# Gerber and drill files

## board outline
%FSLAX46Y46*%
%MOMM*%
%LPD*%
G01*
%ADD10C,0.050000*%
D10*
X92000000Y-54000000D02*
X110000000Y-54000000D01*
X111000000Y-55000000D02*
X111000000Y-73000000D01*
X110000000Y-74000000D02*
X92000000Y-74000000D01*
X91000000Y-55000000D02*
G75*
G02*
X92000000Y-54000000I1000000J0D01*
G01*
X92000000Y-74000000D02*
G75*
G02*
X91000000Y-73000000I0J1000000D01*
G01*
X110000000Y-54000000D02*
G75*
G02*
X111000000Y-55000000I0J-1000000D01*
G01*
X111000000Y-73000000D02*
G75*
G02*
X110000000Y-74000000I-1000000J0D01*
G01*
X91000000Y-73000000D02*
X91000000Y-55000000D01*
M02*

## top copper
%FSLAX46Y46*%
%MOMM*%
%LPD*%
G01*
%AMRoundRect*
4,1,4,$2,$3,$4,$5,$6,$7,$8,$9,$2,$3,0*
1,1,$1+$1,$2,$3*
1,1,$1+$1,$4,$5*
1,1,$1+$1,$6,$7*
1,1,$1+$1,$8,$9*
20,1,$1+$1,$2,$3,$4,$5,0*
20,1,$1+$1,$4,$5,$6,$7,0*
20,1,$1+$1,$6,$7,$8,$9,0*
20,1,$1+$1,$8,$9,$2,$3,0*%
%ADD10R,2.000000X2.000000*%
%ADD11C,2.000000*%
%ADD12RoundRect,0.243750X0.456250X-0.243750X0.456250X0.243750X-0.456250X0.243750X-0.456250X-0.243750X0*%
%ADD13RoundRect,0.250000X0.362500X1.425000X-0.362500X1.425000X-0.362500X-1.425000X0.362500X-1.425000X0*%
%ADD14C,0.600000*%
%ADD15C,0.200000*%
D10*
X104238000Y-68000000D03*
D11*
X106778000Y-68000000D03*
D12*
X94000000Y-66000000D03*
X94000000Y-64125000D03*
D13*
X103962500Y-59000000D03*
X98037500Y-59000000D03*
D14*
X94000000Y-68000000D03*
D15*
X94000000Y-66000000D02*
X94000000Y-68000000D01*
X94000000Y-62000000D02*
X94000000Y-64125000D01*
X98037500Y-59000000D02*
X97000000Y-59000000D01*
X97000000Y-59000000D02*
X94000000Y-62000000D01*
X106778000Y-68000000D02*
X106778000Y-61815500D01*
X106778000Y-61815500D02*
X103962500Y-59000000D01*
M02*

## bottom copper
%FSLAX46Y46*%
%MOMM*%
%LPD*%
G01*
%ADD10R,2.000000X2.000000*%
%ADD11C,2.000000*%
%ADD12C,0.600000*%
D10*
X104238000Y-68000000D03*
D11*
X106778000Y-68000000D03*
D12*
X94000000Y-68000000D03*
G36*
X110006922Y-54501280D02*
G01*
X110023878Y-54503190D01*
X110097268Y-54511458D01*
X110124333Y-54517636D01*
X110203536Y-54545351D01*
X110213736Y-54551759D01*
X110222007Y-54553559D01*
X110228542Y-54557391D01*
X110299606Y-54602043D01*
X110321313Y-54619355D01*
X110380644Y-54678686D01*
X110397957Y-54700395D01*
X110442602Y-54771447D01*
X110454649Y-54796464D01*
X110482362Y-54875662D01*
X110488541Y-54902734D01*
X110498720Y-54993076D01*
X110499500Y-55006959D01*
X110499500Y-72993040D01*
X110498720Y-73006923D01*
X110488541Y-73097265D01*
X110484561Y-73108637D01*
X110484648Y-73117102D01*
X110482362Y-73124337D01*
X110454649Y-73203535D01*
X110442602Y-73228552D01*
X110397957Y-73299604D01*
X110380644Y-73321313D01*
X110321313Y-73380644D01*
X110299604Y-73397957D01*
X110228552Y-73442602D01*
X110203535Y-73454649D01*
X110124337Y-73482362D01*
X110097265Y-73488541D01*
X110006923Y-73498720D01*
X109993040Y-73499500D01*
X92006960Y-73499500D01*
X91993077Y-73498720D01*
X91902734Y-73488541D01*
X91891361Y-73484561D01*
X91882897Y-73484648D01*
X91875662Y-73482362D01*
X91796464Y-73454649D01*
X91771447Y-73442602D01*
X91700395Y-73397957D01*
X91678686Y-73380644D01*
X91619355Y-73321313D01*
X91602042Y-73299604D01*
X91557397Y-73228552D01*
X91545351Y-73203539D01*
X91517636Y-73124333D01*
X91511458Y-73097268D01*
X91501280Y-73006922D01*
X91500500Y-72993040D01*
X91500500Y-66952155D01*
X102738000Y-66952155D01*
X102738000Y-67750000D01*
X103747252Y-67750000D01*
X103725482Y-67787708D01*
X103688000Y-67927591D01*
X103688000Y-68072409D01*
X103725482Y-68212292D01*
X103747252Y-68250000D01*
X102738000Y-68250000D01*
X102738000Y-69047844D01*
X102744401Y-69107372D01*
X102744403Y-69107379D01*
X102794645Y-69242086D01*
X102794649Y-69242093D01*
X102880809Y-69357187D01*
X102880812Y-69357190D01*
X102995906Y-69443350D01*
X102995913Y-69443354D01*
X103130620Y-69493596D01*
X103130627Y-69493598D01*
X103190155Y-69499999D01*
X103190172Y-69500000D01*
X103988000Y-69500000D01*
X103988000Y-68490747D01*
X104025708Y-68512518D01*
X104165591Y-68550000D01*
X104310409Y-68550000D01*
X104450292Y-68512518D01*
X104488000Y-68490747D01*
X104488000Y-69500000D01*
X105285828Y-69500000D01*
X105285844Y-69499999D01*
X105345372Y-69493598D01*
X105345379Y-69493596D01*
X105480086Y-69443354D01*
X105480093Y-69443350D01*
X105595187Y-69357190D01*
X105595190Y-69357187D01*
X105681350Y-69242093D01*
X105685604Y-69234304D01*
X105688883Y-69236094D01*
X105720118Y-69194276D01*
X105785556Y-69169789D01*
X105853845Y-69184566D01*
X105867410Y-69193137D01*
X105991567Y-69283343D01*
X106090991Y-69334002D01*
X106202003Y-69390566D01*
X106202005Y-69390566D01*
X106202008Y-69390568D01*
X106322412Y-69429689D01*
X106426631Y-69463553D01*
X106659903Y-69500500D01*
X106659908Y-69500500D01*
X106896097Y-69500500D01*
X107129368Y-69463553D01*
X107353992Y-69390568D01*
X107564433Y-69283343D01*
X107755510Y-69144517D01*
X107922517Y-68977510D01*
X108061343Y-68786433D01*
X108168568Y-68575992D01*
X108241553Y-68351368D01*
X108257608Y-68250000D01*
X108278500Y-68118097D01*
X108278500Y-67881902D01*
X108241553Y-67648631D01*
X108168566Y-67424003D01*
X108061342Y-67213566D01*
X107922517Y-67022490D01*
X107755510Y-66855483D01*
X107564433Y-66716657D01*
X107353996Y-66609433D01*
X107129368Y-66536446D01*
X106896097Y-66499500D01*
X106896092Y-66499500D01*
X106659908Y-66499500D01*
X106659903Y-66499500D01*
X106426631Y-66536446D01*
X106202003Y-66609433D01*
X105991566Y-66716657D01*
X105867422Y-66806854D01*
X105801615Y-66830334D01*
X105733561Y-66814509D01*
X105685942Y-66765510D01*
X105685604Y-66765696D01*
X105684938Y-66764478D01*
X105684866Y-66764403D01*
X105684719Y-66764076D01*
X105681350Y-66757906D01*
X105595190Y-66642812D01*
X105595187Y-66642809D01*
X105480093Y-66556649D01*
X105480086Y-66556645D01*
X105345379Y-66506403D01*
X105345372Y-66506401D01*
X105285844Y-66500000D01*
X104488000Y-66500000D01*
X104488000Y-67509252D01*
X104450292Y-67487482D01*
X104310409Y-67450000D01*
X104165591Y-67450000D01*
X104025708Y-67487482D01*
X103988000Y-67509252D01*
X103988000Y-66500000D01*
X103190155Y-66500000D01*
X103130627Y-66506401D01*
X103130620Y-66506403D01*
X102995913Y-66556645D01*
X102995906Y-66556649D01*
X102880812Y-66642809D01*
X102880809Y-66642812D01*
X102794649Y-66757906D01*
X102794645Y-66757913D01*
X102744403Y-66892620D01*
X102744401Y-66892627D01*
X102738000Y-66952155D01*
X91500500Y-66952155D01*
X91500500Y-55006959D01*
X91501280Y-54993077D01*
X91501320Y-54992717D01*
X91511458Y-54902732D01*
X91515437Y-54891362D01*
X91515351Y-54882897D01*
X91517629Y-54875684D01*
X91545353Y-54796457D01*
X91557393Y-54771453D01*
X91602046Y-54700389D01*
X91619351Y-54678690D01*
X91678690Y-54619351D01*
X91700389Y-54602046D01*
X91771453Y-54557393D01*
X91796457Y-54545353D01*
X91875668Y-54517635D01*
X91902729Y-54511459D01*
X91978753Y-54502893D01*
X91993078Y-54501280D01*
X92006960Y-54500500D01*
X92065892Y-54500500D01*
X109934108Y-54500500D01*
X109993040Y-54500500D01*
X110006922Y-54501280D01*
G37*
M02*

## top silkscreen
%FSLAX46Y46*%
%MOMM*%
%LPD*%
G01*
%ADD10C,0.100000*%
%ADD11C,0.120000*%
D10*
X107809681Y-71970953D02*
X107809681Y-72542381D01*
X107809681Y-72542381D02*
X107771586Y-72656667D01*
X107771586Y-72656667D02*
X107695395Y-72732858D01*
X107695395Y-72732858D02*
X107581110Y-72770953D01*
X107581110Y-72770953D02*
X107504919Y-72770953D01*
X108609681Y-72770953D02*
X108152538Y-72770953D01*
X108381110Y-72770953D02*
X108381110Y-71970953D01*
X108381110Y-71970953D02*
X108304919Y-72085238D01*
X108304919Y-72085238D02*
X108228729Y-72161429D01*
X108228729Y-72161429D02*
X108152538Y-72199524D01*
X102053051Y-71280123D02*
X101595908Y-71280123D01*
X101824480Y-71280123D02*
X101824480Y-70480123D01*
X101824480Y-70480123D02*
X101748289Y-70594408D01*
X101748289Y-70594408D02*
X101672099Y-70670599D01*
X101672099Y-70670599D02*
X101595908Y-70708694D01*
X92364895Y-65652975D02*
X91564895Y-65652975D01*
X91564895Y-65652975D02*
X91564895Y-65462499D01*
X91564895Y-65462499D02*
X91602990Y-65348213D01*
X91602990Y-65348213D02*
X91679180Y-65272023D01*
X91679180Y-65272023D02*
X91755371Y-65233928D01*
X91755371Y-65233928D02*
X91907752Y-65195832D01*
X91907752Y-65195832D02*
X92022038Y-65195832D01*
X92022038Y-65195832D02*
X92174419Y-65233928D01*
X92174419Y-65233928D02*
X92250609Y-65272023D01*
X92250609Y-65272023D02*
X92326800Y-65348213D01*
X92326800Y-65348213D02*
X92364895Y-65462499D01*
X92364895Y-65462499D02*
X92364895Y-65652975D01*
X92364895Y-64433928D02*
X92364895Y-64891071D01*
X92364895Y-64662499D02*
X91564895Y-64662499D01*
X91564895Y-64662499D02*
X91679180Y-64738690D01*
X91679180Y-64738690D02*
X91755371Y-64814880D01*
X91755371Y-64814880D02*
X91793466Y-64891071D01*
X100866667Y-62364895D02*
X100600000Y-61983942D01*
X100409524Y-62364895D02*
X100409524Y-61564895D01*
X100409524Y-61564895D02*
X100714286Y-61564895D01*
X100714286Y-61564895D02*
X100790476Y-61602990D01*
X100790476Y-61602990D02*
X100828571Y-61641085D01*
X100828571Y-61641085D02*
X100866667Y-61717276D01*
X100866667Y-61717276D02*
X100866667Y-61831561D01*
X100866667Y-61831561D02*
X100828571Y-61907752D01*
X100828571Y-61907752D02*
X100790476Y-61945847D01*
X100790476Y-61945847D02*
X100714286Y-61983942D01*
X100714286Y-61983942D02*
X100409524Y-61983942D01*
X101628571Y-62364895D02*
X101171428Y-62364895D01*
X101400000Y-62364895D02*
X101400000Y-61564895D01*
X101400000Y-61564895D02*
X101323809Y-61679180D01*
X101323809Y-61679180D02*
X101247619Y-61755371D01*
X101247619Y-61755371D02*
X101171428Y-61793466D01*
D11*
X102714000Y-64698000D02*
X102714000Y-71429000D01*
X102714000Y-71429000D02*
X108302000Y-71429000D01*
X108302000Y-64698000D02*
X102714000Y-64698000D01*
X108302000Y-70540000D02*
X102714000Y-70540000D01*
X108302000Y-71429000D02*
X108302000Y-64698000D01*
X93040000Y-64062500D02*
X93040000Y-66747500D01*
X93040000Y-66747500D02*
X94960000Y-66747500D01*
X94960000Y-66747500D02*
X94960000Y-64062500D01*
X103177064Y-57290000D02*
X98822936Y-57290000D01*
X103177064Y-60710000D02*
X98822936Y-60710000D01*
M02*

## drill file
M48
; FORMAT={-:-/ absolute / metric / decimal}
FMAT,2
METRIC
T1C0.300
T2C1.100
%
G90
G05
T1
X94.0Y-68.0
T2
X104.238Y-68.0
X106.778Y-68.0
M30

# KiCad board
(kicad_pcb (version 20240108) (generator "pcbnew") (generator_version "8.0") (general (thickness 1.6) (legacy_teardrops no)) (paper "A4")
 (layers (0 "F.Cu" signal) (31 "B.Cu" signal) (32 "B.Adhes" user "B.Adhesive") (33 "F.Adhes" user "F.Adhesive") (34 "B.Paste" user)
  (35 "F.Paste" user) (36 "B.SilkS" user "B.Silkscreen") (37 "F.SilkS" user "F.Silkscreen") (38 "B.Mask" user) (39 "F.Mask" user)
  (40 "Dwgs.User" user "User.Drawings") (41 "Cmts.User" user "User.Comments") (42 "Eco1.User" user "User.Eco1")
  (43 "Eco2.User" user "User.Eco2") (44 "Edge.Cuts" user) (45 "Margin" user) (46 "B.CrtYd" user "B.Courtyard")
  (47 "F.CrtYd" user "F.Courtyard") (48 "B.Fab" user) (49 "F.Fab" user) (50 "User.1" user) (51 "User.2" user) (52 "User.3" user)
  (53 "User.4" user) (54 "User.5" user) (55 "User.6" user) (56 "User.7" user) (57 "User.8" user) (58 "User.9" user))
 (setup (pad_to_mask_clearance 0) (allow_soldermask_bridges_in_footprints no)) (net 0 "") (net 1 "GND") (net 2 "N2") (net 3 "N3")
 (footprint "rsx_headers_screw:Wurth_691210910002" (layer "F.Cu") (at 105 68)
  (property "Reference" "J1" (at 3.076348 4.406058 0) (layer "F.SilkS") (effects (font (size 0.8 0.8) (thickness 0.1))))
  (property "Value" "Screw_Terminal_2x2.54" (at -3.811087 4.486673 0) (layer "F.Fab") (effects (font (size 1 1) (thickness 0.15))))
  (fp_line (start -2.286 -3.302) (end -2.286 3.429) (stroke (width 0.12) (type solid)) (layer "F.SilkS"))
  (fp_line (start -2.286 3.429) (end 3.302 3.429) (stroke (width 0.12) (type solid)) (layer "F.SilkS"))
  (fp_line (start 3.302 -3.302) (end -2.286 -3.302) (stroke (width 0.12) (type solid)) (layer "F.SilkS"))
  (fp_line (start 3.302 2.54) (end -2.286 2.54) (stroke (width 0.12) (type solid)) (layer "F.SilkS"))
  (fp_line (start 3.302 3.429) (end 3.302 -3.302) (stroke (width 0.12) (type solid)) (layer "F.SilkS"))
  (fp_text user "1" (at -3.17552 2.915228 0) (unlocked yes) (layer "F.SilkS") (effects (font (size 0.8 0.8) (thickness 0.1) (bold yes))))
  (pad "1" thru_hole rect (at -0.762 0) (size 2 2) (drill 1.1) (layers "*.Cu" "*.Mask") (remove_unused_layers no) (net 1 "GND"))
  (pad "2" thru_hole circle (at 1.778 0) (size 2 2) (drill 1.1) (layers "*.Cu" "*.Mask") (remove_unused_layers no) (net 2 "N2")))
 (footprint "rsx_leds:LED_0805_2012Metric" (layer "F.Cu") (at 94 65.0625 90)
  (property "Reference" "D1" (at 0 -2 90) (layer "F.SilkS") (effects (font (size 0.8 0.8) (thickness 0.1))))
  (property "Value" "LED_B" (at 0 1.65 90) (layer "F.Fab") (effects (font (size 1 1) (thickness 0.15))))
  (fp_line (start 1 -0.96) (end -1.685 -0.96) (stroke (width 0.12) (type solid)) (layer "F.SilkS"))
  (fp_line (start -1.685 -0.96) (end -1.685 0.96) (stroke (width 0.12) (type solid)) (layer "F.SilkS"))
  (fp_line (start -1.685 0.96) (end 1 0.96) (stroke (width 0.12) (type solid)) (layer "F.SilkS"))
  (pad "1" smd roundrect (at -0.9375 0 90) (size 0.975 1.4) (layers "F.Cu" "F.Paste" "F.Mask") (roundrect_rratio 0.25) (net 1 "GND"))
  (pad "2" smd roundrect (at 0.9375 0 90) (size 0.975 1.4) (layers "F.Cu" "F.Paste" "F.Mask") (roundrect_rratio 0.25) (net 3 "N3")))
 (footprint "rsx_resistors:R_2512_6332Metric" (layer "F.Cu") (at 101 59 180)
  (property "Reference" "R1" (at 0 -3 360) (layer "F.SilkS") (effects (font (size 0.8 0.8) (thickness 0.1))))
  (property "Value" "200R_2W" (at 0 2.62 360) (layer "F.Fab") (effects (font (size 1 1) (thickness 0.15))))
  (fp_line (start -2.177064 1.71) (end 2.177064 1.71) (stroke (width 0.12) (type solid)) (layer "F.SilkS"))
  (fp_line (start -2.177064 -1.71) (end 2.177064 -1.71) (stroke (width 0.12) (type solid)) (layer "F.SilkS"))
  (pad "1" smd roundrect (at -2.9625 0 180) (size 1.225 3.35) (layers "F.Cu" "F.Paste" "F.Mask") (roundrect_rratio 0.204082) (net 2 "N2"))
  (pad "2" smd roundrect (at 2.9625 0 180) (size 1.225 3.35) (layers "F.Cu" "F.Paste" "F.Mask") (roundrect_rratio 0.204082) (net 3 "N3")))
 (gr_line (start 92 54) (end 110 54) (stroke (width 0.05) (type default)) (layer "Edge.Cuts"))
 (gr_line (start 111 55) (end 111 73) (stroke (width 0.05) (type default)) (layer "Edge.Cuts"))
 (gr_line (start 110 74) (end 92 74) (stroke (width 0.05) (type default)) (layer "Edge.Cuts"))
 (gr_arc (start 91 55) (mid 91.292893 54.292893) (end 92 54) (stroke (width 0.05) (type default)) (layer "Edge.Cuts"))
 (gr_arc (start 92 74) (mid 91.292893 73.707107) (end 91 73) (stroke (width 0.05) (type default)) (layer "Edge.Cuts"))
 (gr_arc (start 110 54) (mid 110.707107 54.292893) (end 111 55) (stroke (width 0.05) (type default)) (layer "Edge.Cuts"))
 (gr_arc (start 111 73) (mid 110.707107 73.707107) (end 110 74) (stroke (width 0.05) (type default)) (layer "Edge.Cuts"))
 (gr_line (start 91 73) (end 91 55) (stroke (width 0.05) (type default)) (layer "Edge.Cuts"))
 (segment (start 94 66) (end 94 68) (width 0.2) (layer "F.Cu") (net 1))
 (via (at 94 68) (size 0.6) (drill 0.3) (layers "F.Cu" "B.Cu") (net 1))
 (segment (start 94 62) (end 94 64.125) (width 0.2) (layer "F.Cu") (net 3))
 (segment (start 98.0375 59) (end 97 59) (width 0.2) (layer "F.Cu") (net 3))
 (segment (start 97 59) (end 94 62) (width 0.2) (layer "F.Cu") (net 3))
 (segment (start 106.778 68) (end 106.778 61.8155) (width 0.2) (layer "F.Cu") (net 2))
 (segment (start 106.778 61.8155) (end 103.9625 59) (width 0.2) (layer "F.Cu") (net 2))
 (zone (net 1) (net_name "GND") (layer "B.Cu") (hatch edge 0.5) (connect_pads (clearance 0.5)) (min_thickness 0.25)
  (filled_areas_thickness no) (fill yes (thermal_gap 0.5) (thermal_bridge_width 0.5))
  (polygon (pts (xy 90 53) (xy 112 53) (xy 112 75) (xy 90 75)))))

